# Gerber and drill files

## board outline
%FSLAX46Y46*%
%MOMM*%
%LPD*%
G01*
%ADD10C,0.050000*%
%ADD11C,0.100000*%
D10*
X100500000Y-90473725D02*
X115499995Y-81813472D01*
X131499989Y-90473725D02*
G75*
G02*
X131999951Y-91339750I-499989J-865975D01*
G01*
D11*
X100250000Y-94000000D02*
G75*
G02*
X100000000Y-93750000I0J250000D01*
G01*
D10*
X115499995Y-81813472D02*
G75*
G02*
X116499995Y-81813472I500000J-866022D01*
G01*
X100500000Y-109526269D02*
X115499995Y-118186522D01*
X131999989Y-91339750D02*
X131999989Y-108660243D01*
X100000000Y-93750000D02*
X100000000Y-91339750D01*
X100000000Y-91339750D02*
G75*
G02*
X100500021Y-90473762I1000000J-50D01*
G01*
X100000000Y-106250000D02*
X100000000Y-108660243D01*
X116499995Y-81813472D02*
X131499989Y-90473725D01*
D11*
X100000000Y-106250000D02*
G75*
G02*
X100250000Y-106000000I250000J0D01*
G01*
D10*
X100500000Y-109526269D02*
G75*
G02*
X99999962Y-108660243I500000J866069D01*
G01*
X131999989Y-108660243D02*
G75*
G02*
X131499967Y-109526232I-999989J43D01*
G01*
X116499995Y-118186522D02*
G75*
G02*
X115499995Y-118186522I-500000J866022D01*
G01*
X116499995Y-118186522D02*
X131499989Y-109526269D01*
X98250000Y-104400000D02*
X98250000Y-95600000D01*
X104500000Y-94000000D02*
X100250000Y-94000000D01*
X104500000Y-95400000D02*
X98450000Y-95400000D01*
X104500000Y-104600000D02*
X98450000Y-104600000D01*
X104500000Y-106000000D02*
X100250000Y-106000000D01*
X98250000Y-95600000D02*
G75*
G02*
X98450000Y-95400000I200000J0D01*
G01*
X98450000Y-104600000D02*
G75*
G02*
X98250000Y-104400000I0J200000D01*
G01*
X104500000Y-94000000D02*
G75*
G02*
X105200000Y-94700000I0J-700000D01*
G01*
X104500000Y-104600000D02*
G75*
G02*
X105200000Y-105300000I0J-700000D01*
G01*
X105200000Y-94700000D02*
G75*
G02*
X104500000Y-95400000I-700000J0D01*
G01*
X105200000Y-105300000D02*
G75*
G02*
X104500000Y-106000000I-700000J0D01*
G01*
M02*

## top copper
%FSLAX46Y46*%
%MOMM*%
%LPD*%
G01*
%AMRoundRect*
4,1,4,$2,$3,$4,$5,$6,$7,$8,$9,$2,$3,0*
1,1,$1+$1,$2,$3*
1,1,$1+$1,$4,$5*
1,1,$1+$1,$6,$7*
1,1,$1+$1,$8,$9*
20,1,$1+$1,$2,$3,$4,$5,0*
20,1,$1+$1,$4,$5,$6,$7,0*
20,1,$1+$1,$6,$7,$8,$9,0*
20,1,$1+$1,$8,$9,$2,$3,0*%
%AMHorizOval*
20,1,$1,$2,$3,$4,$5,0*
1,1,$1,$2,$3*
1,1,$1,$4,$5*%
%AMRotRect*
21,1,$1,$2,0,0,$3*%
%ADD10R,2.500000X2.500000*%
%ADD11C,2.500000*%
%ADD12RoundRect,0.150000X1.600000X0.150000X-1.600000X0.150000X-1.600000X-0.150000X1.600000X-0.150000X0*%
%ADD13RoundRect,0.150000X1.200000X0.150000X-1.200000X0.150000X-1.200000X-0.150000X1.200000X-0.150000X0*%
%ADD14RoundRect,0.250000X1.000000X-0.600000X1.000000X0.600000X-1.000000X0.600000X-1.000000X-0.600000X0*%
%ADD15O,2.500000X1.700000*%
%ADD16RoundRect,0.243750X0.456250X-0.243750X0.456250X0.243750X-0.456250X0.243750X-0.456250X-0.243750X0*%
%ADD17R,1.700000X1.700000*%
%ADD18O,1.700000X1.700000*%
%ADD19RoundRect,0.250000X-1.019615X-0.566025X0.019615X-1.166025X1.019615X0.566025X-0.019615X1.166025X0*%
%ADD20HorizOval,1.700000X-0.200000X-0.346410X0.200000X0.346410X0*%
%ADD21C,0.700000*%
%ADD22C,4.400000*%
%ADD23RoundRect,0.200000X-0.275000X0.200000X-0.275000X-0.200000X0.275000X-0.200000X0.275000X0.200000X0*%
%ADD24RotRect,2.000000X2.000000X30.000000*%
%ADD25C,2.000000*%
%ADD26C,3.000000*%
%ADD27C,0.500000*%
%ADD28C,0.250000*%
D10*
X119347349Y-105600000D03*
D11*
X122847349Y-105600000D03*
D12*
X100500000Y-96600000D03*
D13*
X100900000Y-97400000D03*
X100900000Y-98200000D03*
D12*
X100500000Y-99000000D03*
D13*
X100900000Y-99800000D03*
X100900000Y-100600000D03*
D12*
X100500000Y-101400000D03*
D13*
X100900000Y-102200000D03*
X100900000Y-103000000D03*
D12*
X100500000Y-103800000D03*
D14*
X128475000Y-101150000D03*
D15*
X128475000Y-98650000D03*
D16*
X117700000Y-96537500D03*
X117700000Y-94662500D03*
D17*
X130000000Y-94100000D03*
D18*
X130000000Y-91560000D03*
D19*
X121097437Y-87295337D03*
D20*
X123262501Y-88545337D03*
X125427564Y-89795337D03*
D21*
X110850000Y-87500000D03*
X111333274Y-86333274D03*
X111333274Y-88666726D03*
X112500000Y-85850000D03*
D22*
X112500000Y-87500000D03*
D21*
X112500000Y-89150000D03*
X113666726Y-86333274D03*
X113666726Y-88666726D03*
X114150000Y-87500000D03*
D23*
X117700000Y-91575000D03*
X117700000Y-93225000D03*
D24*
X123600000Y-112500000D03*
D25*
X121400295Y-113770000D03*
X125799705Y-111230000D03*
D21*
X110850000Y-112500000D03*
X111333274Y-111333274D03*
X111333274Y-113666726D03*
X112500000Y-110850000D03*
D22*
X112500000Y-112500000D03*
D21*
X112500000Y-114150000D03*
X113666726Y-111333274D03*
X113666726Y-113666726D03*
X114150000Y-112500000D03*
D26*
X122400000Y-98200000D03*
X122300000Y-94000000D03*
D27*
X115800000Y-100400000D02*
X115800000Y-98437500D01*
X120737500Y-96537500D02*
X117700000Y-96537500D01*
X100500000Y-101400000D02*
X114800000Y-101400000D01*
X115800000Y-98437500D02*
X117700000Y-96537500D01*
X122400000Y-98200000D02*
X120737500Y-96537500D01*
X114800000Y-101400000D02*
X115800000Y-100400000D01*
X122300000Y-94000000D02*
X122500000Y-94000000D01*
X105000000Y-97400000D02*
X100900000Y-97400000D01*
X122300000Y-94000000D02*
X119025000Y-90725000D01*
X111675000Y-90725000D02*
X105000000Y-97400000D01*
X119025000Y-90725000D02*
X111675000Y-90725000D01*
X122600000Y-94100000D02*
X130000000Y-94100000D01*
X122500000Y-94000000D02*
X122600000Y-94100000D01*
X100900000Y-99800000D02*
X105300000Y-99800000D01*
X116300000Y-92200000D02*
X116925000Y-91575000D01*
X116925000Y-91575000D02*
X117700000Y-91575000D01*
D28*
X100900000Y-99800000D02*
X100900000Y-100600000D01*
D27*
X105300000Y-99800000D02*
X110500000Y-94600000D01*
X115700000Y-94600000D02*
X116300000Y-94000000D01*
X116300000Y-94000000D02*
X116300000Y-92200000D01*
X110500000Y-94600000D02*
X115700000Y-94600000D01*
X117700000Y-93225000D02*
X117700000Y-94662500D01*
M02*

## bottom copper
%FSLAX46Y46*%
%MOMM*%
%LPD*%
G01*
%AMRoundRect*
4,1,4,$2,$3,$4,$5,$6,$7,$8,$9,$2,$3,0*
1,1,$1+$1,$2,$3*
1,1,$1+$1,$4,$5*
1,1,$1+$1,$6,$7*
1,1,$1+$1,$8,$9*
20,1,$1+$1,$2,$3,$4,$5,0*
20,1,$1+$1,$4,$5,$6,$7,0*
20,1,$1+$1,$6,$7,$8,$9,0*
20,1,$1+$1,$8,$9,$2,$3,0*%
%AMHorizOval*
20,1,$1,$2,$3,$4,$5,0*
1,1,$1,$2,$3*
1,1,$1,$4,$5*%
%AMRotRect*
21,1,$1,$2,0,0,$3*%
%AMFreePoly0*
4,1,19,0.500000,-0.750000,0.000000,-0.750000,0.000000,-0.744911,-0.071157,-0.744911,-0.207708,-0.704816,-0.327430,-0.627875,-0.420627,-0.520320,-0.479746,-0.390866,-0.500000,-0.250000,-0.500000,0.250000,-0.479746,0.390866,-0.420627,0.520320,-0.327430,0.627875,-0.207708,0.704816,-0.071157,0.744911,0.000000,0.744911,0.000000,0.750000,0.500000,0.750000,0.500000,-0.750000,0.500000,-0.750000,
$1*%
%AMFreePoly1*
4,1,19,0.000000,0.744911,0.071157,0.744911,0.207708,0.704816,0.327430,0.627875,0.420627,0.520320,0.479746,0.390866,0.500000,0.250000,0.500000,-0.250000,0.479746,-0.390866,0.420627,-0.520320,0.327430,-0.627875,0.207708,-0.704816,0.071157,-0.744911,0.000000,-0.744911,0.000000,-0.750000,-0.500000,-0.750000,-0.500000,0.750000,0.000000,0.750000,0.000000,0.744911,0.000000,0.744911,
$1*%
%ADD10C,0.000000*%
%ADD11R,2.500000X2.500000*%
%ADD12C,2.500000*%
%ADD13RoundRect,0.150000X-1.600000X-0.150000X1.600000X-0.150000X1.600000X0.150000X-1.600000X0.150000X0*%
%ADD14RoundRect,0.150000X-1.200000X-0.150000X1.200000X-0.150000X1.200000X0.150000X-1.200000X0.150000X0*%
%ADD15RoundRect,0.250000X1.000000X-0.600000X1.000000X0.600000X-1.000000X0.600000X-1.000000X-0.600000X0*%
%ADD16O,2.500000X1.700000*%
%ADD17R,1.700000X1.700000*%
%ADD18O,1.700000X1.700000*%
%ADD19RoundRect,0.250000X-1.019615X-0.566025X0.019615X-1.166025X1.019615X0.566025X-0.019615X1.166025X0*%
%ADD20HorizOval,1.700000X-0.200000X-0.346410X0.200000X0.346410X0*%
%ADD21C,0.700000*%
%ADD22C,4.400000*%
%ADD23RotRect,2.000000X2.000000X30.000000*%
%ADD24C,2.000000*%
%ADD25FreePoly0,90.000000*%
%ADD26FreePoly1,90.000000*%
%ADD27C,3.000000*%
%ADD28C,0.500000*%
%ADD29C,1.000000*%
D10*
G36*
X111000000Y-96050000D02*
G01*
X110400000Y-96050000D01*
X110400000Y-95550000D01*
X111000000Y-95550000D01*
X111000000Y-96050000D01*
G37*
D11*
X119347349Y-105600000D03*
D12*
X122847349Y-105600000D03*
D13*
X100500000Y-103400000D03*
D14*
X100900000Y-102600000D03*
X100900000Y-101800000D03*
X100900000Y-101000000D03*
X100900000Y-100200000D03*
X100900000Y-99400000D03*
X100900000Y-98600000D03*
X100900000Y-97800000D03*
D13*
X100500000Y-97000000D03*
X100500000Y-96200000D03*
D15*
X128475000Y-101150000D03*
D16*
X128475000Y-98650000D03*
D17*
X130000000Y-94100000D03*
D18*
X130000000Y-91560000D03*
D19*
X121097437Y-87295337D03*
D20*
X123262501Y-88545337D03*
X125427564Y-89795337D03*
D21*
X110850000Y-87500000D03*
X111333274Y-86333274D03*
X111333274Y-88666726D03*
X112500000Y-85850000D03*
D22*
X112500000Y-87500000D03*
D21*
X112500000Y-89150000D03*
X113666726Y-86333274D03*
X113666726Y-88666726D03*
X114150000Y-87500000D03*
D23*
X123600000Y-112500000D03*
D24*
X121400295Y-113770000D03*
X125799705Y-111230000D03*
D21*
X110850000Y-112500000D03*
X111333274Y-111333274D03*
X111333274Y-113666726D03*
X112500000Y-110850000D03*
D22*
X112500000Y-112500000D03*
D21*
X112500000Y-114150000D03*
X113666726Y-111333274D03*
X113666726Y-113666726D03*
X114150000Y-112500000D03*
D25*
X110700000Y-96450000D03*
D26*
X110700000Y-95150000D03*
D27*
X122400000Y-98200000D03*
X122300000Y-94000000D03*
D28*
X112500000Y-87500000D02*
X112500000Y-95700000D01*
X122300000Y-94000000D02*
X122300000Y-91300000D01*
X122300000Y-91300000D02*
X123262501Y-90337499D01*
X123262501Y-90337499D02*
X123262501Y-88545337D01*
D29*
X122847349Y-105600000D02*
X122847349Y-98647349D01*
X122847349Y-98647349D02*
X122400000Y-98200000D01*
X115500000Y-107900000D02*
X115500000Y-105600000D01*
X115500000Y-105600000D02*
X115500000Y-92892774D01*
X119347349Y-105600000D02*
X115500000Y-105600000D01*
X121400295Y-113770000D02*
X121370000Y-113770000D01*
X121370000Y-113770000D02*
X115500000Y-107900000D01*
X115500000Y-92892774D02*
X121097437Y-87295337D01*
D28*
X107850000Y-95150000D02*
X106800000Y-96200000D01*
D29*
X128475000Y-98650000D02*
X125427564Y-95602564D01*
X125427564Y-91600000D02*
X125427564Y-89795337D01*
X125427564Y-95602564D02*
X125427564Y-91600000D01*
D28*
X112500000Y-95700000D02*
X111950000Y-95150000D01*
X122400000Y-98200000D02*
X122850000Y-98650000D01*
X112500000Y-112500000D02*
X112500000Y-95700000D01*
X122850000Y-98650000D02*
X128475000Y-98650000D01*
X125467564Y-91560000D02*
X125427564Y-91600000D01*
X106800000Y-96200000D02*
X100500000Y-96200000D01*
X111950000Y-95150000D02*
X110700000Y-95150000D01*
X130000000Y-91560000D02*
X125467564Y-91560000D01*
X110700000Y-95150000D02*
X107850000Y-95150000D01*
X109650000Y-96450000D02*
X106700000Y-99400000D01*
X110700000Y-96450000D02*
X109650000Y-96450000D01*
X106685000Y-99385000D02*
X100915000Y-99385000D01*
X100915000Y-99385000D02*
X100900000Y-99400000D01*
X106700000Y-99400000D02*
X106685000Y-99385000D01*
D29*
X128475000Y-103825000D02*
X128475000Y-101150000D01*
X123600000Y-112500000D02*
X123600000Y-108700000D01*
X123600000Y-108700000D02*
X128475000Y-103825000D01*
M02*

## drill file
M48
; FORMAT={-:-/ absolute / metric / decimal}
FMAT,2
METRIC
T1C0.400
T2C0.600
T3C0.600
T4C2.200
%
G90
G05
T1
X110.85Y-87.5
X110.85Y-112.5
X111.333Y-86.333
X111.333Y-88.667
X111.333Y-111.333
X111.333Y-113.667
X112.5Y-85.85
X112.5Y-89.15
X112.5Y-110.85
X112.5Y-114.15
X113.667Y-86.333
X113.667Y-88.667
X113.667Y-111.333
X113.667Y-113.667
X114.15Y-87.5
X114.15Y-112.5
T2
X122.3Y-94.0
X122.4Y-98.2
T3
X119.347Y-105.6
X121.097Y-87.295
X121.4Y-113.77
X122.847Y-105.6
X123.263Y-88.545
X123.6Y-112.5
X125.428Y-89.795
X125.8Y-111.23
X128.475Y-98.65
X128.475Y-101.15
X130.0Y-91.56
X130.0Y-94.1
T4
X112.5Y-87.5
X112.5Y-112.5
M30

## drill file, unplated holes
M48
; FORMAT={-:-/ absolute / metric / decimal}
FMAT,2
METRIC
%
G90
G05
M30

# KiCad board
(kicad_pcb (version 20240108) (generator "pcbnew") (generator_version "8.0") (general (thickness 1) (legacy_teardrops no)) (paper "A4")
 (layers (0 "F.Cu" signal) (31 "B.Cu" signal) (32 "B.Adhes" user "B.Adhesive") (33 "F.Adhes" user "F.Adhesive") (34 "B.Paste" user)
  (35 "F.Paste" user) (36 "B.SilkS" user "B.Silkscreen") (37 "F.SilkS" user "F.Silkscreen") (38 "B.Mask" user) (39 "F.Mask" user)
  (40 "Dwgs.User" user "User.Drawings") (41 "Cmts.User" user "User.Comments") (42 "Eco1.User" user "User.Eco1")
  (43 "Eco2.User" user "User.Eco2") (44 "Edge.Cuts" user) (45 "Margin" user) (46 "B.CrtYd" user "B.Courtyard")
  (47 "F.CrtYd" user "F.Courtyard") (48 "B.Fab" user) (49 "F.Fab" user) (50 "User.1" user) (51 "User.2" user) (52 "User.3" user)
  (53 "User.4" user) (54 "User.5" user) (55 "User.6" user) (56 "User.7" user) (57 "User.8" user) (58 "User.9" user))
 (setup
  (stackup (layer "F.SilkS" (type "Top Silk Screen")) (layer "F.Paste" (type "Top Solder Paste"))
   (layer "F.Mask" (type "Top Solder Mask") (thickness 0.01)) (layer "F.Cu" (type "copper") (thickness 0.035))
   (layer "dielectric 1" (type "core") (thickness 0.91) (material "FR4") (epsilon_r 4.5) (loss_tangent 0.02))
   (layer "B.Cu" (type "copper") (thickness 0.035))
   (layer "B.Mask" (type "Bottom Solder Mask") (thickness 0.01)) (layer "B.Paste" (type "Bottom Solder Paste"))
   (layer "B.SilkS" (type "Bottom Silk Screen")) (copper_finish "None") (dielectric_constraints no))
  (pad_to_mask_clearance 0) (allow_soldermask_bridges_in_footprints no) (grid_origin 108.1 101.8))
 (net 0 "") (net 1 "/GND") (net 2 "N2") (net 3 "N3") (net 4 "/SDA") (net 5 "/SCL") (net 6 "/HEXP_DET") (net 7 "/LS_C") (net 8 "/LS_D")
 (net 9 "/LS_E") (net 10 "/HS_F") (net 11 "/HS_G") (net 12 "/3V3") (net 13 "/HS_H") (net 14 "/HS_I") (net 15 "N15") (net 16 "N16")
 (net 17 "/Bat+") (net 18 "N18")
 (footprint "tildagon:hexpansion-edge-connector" (layer "F.Cu") (at 98.25 100)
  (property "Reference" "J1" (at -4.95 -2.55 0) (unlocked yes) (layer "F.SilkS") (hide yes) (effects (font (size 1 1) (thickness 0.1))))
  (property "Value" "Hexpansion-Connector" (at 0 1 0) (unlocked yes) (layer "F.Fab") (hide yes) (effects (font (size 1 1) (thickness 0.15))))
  (fp_line (start 0 4.4) (end 0 -4.4) (stroke (width 0.05) (type solid)) (layer "Edge.Cuts"))
  (fp_line (start 6.25 -6) (end 2 -6) (stroke (width 0.05) (type solid)) (layer "Edge.Cuts"))
  (fp_line (start 6.25 -4.6) (end 0.2 -4.6) (stroke (width 0.05) (type solid)) (layer "Edge.Cuts"))
  (fp_line (start 6.25 4.6) (end 0.2 4.6) (stroke (width 0.05) (type solid)) (layer "Edge.Cuts"))
  (fp_line (start 6.25 6) (end 2 6) (stroke (width 0.05) (type solid)) (layer "Edge.Cuts"))
  (fp_arc (start 0 -4.4) (mid 0.058579 -4.541421) (end 0.2 -4.6) (stroke (width 0.05) (type default)) (layer "Edge.Cuts"))
  (fp_arc (start 0.2 4.6) (mid 0.058579 4.541421) (end 0 4.4) (stroke (width 0.05) (type default)) (layer "Edge.Cuts"))
  (fp_arc (start 6.25 -6) (mid 6.744975 -5.794975) (end 6.95 -5.3) (stroke (width 0.05) (type default)) (layer "Edge.Cuts"))
  (fp_arc (start 6.25 4.6) (mid 6.744975 4.805025) (end 6.95 5.3) (stroke (width 0.05) (type default)) (layer "Edge.Cuts"))
  (fp_arc (start 6.95 -5.3) (mid 6.744975 -4.805025) (end 6.25 -4.6) (stroke (width 0.05) (type default)) (layer "Edge.Cuts"))
  (fp_arc (start 6.95 5.3) (mid 6.744975 5.794975) (end 6.25 6) (stroke (width 0.05) (type default)) (layer "Edge.Cuts"))
  (pad "1" smd roundrect (at 2.25 3.4) (size 3.5 0.6) (layers "B.Cu" "B.Mask") (roundrect_rratio 0.25) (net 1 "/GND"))
  (pad "2" smd roundrect (at 2.65 2.6) (size 2.7 0.6) (layers "B.Cu" "B.Mask") (roundrect_rratio 0.25) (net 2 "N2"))
  (pad "3" smd roundrect (at 2.65 1.8) (size 2.7 0.6) (layers "B.Cu" "B.Mask") (roundrect_rratio 0.25) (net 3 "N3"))
  (pad "4" smd roundrect (at 2.65 1) (size 2.7 0.6) (layers "B.Cu" "B.Mask") (roundrect_rratio 0.25) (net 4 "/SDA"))
  (pad "5" smd roundrect (at 2.65 0.2) (size 2.7 0.6) (layers "B.Cu" "B.Mask") (roundrect_rratio 0.25) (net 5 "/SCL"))
  (pad "6" smd roundrect (at 2.65 -0.6) (size 2.7 0.6) (layers "B.Cu" "B.Mask") (roundrect_rratio 0.25) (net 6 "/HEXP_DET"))
  (pad "7" smd roundrect (at 2.65 -1.4) (size 2.7 0.6) (layers "B.Cu" "B.Mask") (roundrect_rratio 0.25) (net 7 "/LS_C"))
  (pad "8" smd roundrect (at 2.65 -2.2) (size 2.7 0.6) (layers "B.Cu" "B.Mask") (roundrect_rratio 0.25) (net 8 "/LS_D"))
  (pad "9" smd roundrect (at 2.25 -3) (size 3.5 0.6) (layers "B.Cu" "B.Mask") (roundrect_rratio 0.25) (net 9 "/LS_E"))
  (pad "10" smd roundrect (at 2.25 -3.8) (size 3.5 0.6) (layers "B.Cu" "B.Mask") (roundrect_rratio 0.25) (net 1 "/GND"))
  (pad "11" smd roundrect (at 2.25 -3.4 180) (size 3.5 0.6) (layers "F.Cu" "F.Mask") (roundrect_rratio 0.25) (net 1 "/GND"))
  (pad "12" smd roundrect (at 2.65 -2.6 180) (size 2.7 0.6) (layers "F.Cu" "F.Mask") (roundrect_rratio 0.25) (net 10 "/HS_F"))
  (pad "13" smd roundrect (at 2.65 -1.8 180) (size 2.7 0.6) (layers "F.Cu" "F.Mask") (roundrect_rratio 0.25) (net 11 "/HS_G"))
  (pad "14" smd roundrect (at 2.25 -1 180) (size 3.5 0.6) (layers "F.Cu" "F.Mask") (roundrect_rratio 0.25) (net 1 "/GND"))
  (pad "15" smd roundrect (at 2.65 -0.2 180) (size 2.7 0.6) (layers "F.Cu" "F.Mask") (roundrect_rratio 0.25) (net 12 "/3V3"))
  (pad "16" smd roundrect (at 2.65 0.6 180) (size 2.7 0.6) (layers "F.Cu" "F.Mask") (roundrect_rratio 0.25) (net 12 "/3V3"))
  (pad "17" smd roundrect (at 2.25 1.4 180) (size 3.5 0.6) (layers "F.Cu" "F.Mask") (roundrect_rratio 0.25) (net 1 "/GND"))
  (pad "18" smd roundrect (at 2.65 2.2 180) (size 2.7 0.6) (layers "F.Cu" "F.Mask") (roundrect_rratio 0.25) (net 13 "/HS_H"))
  (pad "19" smd roundrect (at 2.65 3 180) (size 2.7 0.6) (layers "F.Cu" "F.Mask") (roundrect_rratio 0.25) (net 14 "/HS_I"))
  (pad "20" smd roundrect (at 2.25 3.8 180) (size 3.5 0.6) (layers "F.Cu" "F.Mask") (roundrect_rratio 0.25) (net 1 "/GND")))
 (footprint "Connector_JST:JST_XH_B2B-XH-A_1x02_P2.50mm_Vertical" (layer "F.Cu") (at 128.475 101.15 90)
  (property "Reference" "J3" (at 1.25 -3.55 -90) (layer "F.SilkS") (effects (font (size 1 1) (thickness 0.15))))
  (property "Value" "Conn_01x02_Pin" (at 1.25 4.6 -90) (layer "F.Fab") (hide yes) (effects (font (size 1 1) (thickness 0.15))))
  (pad "1" thru_hole roundrect (at 0 0 90) (size 1.7 2.5) (drill 0.6) (layers "*.Cu" "*.Mask") (remove_unused_layers no)
   (roundrect_rratio 0.147059) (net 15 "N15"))
  (pad "2" thru_hole oval (at 2.5 0 90) (size 1.7 2.5) (drill 0.6) (layers "*.Cu" "*.Mask") (remove_unused_layers no) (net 1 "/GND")))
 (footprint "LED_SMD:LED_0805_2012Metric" (layer "F.Cu") (at 117.7 95.6 90)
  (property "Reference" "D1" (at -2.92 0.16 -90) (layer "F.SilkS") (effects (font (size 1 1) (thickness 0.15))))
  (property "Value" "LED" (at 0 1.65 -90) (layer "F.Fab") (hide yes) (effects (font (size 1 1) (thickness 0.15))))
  (pad "1" smd roundrect (at -0.9375 0 90) (size 0.975 1.4) (layers "F.Cu" "F.Paste" "F.Mask") (roundrect_rratio 0.25) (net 1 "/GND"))
  (pad "2" smd roundrect (at 0.9375 0 90) (size 0.975 1.4) (layers "F.Cu" "F.Paste" "F.Mask") (roundrect_rratio 0.25) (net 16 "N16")))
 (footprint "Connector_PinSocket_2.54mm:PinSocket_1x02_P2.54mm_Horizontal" (layer "F.Cu") (at 130 94.1 180)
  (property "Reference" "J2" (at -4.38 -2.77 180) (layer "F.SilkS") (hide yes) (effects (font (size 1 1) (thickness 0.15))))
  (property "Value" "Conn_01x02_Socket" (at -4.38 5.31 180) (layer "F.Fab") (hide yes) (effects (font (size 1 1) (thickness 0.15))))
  (pad "1" thru_hole rect (at 0 0 180) (size 1.7 1.7) (drill 0.6) (layers "*.Cu" "*.Mask") (remove_unused_layers no) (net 10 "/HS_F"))
  (pad "2" thru_hole oval (at 0 2.54 180) (size 1.7 1.7) (drill 0.6) (layers "*.Cu" "*.Mask") (remove_unused_layers no) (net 1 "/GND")))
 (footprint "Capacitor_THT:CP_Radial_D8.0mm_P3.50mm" (layer "F.Cu") (at 119.347349 105.6)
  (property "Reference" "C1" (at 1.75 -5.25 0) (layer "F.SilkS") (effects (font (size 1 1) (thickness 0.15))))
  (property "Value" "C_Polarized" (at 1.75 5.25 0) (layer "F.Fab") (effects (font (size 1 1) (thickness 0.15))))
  (pad "1" thru_hole rect (at 0 0) (size 2.5 2.5) (drill 0.6) (layers "*.Cu" "*.Mask") (remove_unused_layers no) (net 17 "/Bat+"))
  (pad "2" thru_hole circle (at 3.5 0) (size 2.5 2.5) (drill 0.6) (layers "*.Cu" "*.Mask") (remove_unused_layers no) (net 1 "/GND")))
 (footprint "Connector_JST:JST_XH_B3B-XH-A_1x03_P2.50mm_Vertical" (layer "F.Cu") (at 121.097437 87.295337 -30)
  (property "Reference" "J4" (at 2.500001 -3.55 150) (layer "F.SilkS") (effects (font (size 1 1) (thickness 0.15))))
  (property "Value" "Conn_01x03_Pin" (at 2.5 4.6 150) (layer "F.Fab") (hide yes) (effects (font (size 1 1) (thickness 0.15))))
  (pad "1" thru_hole roundrect (at 0 0 330) (size 1.7 2.5) (drill 0.6) (layers "*.Cu" "*.Mask") (remove_unused_layers no)
   (roundrect_rratio 0.147059) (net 17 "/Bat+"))
  (pad "2" thru_hole oval (at 2.5 0 330) (size 1.7 2.5) (drill 0.6) (layers "*.Cu" "*.Mask") (remove_unused_layers no) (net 10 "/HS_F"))
  (pad "3" thru_hole oval (at 5 0 330) (size 1.7 2.5) (drill 0.6) (layers "*.Cu" "*.Mask") (remove_unused_layers no) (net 1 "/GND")))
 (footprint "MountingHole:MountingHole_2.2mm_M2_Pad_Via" (layer "F.Cu") (at 112.5 87.5)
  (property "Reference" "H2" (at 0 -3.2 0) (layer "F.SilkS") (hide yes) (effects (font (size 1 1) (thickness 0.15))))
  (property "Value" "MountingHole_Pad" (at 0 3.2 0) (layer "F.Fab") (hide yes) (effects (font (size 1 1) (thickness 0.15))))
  (pad "1" thru_hole circle (at -1.65 0) (size 0.7 0.7) (drill 0.4) (layers "*.Cu" "*.Mask") (remove_unused_layers no) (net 1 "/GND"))
  (pad "1" thru_hole circle (at -1.166726 -1.166726) (size 0.7 0.7) (drill 0.4) (layers "*.Cu" "*.Mask") (remove_unused_layers no)
   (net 1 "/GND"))
  (pad "1" thru_hole circle (at -1.166726 1.166726) (size 0.7 0.7) (drill 0.4) (layers "*.Cu" "*.Mask") (remove_unused_layers no)
   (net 1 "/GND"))
  (pad "1" thru_hole circle (at 0 -1.65) (size 0.7 0.7) (drill 0.4) (layers "*.Cu" "*.Mask") (remove_unused_layers no) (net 1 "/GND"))
  (pad "1" thru_hole circle (at 0 0) (size 4.4 4.4) (drill 2.2) (layers "*.Cu" "*.Mask") (remove_unused_layers no) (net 1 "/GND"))
  (pad "1" thru_hole circle (at 0 1.65) (size 0.7 0.7) (drill 0.4) (layers "*.Cu" "*.Mask") (remove_unused_layers no) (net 1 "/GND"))
  (pad "1" thru_hole circle (at 1.166726 -1.166726) (size 0.7 0.7) (drill 0.4) (layers "*.Cu" "*.Mask") (remove_unused_layers no)
   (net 1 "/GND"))
  (pad "1" thru_hole circle (at 1.166726 1.166726) (size 0.7 0.7) (drill 0.4) (layers "*.Cu" "*.Mask") (remove_unused_layers no)
   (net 1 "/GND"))
  (pad "1" thru_hole circle (at 1.65 0) (size 0.7 0.7) (drill 0.4) (layers "*.Cu" "*.Mask") (remove_unused_layers no) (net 1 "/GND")))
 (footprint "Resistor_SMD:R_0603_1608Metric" (layer "F.Cu") (at 117.7 92.4 -90)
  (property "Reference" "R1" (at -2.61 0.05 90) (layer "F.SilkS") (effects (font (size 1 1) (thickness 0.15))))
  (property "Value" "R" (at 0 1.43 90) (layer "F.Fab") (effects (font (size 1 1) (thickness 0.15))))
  (pad "1" smd roundrect (at -0.825 0 270) (size 0.8 0.95) (layers "F.Cu" "F.Paste" "F.Mask") (roundrect_rratio 0.25) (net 12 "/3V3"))
  (pad "2" smd roundrect (at 0.825 0 270) (size 0.8 0.95) (layers "F.Cu" "F.Paste" "F.Mask") (roundrect_rratio 0.25) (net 16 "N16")))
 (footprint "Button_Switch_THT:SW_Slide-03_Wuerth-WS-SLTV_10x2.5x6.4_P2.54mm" (layer "F.Cu") (at 123.6 112.5 30)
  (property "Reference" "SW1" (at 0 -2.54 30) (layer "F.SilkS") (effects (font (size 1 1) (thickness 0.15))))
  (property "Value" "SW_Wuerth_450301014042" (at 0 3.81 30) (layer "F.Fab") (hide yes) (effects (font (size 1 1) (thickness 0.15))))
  (pad "1" thru_hole rect (at 0 0 30) (size 2 2) (drill 0.6) (layers "*.Cu" "*.Mask") (remove_unused_layers no) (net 15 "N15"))
  (pad "2" thru_hole circle (at -2.54 0 30) (size 2 2) (drill 0.6) (layers "*.Cu" "*.Mask") (remove_unused_layers no) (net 17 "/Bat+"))
  (pad "3" thru_hole circle (at 2.54 0 30) (size 2 2) (drill 0.6) (layers "*.Cu" "*.Mask") (remove_unused_layers no) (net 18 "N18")))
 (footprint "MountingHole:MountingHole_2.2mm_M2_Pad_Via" (layer "F.Cu") (at 112.5 112.5)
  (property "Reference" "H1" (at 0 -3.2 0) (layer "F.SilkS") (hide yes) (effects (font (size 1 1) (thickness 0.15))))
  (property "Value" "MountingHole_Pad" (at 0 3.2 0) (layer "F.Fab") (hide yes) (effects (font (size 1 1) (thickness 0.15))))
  (pad "1" thru_hole circle (at -1.65 0) (size 0.7 0.7) (drill 0.4) (layers "*.Cu" "*.Mask") (remove_unused_layers no) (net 1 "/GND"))
  (pad "1" thru_hole circle (at -1.166726 -1.166726) (size 0.7 0.7) (drill 0.4) (layers "*.Cu" "*.Mask") (remove_unused_layers no)
   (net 1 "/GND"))
  (pad "1" thru_hole circle (at -1.166726 1.166726) (size 0.7 0.7) (drill 0.4) (layers "*.Cu" "*.Mask") (remove_unused_layers no)
   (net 1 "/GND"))
  (pad "1" thru_hole circle (at 0 -1.65) (size 0.7 0.7) (drill 0.4) (layers "*.Cu" "*.Mask") (remove_unused_layers no) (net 1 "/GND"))
  (pad "1" thru_hole circle (at 0 0) (size 4.4 4.4) (drill 2.2) (layers "*.Cu" "*.Mask") (remove_unused_layers no) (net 1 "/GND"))
  (pad "1" thru_hole circle (at 0 1.65) (size 0.7 0.7) (drill 0.4) (layers "*.Cu" "*.Mask") (remove_unused_layers no) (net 1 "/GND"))
  (pad "1" thru_hole circle (at 1.166726 -1.166726) (size 0.7 0.7) (drill 0.4) (layers "*.Cu" "*.Mask") (remove_unused_layers no)
   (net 1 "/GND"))
  (pad "1" thru_hole circle (at 1.166726 1.166726) (size 0.7 0.7) (drill 0.4) (layers "*.Cu" "*.Mask") (remove_unused_layers no)
   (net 1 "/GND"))
  (pad "1" thru_hole circle (at 1.65 0) (size 0.7 0.7) (drill 0.4) (layers "*.Cu" "*.Mask") (remove_unused_layers no) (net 1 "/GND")))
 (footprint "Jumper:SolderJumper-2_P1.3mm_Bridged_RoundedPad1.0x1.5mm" (layer "B.Cu") (at 110.7 95.8 90)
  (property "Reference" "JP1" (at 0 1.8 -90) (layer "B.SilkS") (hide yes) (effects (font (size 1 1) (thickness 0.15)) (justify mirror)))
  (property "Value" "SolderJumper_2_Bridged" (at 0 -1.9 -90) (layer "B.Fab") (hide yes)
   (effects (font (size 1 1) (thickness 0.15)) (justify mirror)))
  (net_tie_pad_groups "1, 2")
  (fp_poly (pts (xy 0.25 0.3) (xy -0.25 0.3) (xy -0.25 -0.3) (xy 0.25 -0.3)) (stroke (width 0) (type solid)) (fill solid) (layer "B.Cu"))
  (pad "1" smd custom (at -0.65 0 90) (size 1 0.5) (layers "B.Cu" "B.Mask") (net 6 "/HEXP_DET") (zone_connect 2)
   (options (clearance outline) (anchor rect)) (primitives))
  (pad "2" smd custom (at 0.65 0 90) (size 1 0.5) (layers "B.Cu" "B.Mask") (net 1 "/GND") (zone_connect 2)
   (options (clearance outline) (anchor rect)) (primitives)))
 (gr_line (start 100.5 90.473725) (end 115.499995 81.813472) (stroke (width 0.05) (type solid)) (layer "Edge.Cuts"))
 (gr_arc (start 131.499989 90.473725) (mid 131.866015 90.83975) (end 131.999989 91.33975) (stroke (width 0.05) (type solid))
  (layer "Edge.Cuts"))
 (gr_arc (start 100.25 94) (mid 100.073223 93.926777) (end 100 93.75) (stroke (width 0.1) (type default)) (layer "Edge.Cuts"))
 (gr_arc (start 115.499995 81.813472) (mid 115.999995 81.679497) (end 116.499995 81.813472) (stroke (width 0.05) (type solid))
  (layer "Edge.Cuts"))
 (gr_line (start 100.5 109.526269) (end 115.499995 118.186522) (stroke (width 0.05) (type solid)) (layer "Edge.Cuts"))
 (gr_line (start 131.999989 91.33975) (end 131.999989 108.660243) (stroke (width 0.05) (type solid)) (layer "Edge.Cuts"))
 (gr_line (start 100 93.75) (end 100 91.33975) (stroke (width 0.05) (type solid)) (layer "Edge.Cuts"))
 (gr_arc (start 100 91.33975) (mid 100.133975 90.83975) (end 100.5 90.473725) (stroke (width 0.05) (type solid)) (layer "Edge.Cuts"))
 (gr_line (start 100 106.25) (end 100 108.660243) (stroke (width 0.05) (type solid)) (layer "Edge.Cuts"))
 (gr_line (start 116.499995 81.813472) (end 131.499989 90.473725) (stroke (width 0.05) (type solid)) (layer "Edge.Cuts"))
 (gr_arc (start 100 106.25) (mid 100.073223 106.073223) (end 100.25 106) (stroke (width 0.1) (type default)) (layer "Edge.Cuts"))
 (gr_arc (start 100.5 109.526269) (mid 100.133975 109.160243) (end 100 108.660243) (stroke (width 0.05) (type solid)) (layer "Edge.Cuts"))
 (gr_arc (start 131.999989 108.660243) (mid 131.866015 109.160243) (end 131.499989 109.526269) (stroke (width 0.05) (type solid))
  (layer "Edge.Cuts"))
 (gr_arc (start 116.499995 118.186522) (mid 115.999995 118.320497) (end 115.499995 118.186522) (stroke (width 0.05) (type solid))
  (layer "Edge.Cuts"))
 (gr_line (start 116.499995 118.186522) (end 131.499989 109.526269) (stroke (width 0.05) (type solid)) (layer "Edge.Cuts"))
 (segment (start 115.8 100.4) (end 115.8 98.4375) (width 0.5) (layer "F.Cu") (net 1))
 (segment (start 120.7375 96.5375) (end 117.7 96.5375) (width 0.5) (layer "F.Cu") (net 1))
 (segment (start 100.5 101.4) (end 114.8 101.4) (width 0.5) (layer "F.Cu") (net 1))
 (segment (start 115.8 98.4375) (end 117.7 96.5375) (width 0.5) (layer "F.Cu") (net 1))
 (segment (start 122.4 98.2) (end 120.7375 96.5375) (width 0.5) (layer "F.Cu") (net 1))
 (segment (start 114.8 101.4) (end 115.8 100.4) (width 0.5) (layer "F.Cu") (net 1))
 (via (at 122.4 98.2) (size 3) (drill 0.6) (layers "F.Cu" "B.Cu") (free yes) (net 1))
 (segment (start 107.85 95.15) (end 106.8 96.2) (width 0.5) (layer "B.Cu") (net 1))
 (segment (start 128.475 98.65) (end 125.427564 95.602564) (width 1) (layer "B.Cu") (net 1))
 (segment (start 125.427564 91.6) (end 125.427564 89.795337) (width 1) (layer "B.Cu") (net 1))
 (segment (start 125.427564 95.602564) (end 125.427564 91.6) (width 1) (layer "B.Cu") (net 1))
 (segment (start 122.847349 98.647349) (end 122.4 98.2) (width 1) (layer "B.Cu") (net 1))
 (segment (start 112.5 95.7) (end 111.95 95.15) (width 0.5) (layer "B.Cu") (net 1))
 (segment (start 122.4 98.2) (end 122.85 98.65) (width 0.5) (layer "B.Cu") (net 1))
 (segment (start 112.5 112.5) (end 112.5 95.7) (width 0.5) (layer "B.Cu") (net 1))
 (segment (start 112.5 87.5) (end 112.5 95.7) (width 0.5) (layer "B.Cu") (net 1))
 (segment (start 122.847349 105.6) (end 122.847349 98.647349) (width 1) (layer "B.Cu") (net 1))
 (segment (start 122.85 98.65) (end 128.475 98.65) (width 0.5) (layer "B.Cu") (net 1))
 (segment (start 125.467564 91.56) (end 125.427564 91.6) (width 0.5) (layer "B.Cu") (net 1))
 (segment (start 106.8 96.2) (end 100.5 96.2) (width 0.5) (layer "B.Cu") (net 1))
 (segment (start 111.95 95.15) (end 110.7 95.15) (width 0.5) (layer "B.Cu") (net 1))
 (segment (start 130 91.56) (end 125.467564 91.56) (width 0.5) (layer "B.Cu") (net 1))
 (segment (start 110.7 95.15) (end 107.85 95.15) (width 0.5) (layer "B.Cu") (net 1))
 (segment (start 122.3 94) (end 122.5 94) (width 0.5) (layer "F.Cu") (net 10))
 (segment (start 105 97.4) (end 100.9 97.4) (width 0.5) (layer "F.Cu") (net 10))
 (segment (start 122.3 94) (end 119.025 90.725) (width 0.5) (layer "F.Cu") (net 10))
 (segment (start 111.675 90.725) (end 105 97.4) (width 0.5) (layer "F.Cu") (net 10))
 (segment (start 119.025 90.725) (end 111.675 90.725) (width 0.5) (layer "F.Cu") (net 10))
 (segment (start 122.6 94.1) (end 130 94.1) (width 0.5) (layer "F.Cu") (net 10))
 (segment (start 122.5 94) (end 122.6 94.1) (width 0.5) (layer "F.Cu") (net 10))
 (via (at 122.3 94) (size 3) (drill 0.6) (layers "F.Cu" "B.Cu") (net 10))
 (segment (start 122.3 91.3) (end 123.262501 90.337499) (width 0.5) (layer "B.Cu") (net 10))
 (segment (start 122.3 94) (end 122.3 91.3) (width 0.5) (layer "B.Cu") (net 10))
 (segment (start 123.262501 90.337499) (end 123.262501 88.545337) (width 0.5) (layer "B.Cu") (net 10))
 (segment (start 100.9 99.8) (end 105.3 99.8) (width 0.5) (layer "F.Cu") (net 12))
 (segment (start 116.3 92.2) (end 116.925 91.575) (width 0.5) (layer "F.Cu") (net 12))
 (segment (start 116.925 91.575) (end 117.7 91.575) (width 0.5) (layer "F.Cu") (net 12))
 (segment (start 100.9 99.8) (end 100.9 100.6) (width 0.25) (layer "F.Cu") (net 12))
 (segment (start 105.3 99.8) (end 110.5 94.6) (width 0.5) (layer "F.Cu") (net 12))
 (segment (start 115.7 94.6) (end 116.3 94) (width 0.5) (layer "F.Cu") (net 12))
 (segment (start 116.3 94) (end 116.3 92.2) (width 0.5) (layer "F.Cu") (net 12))
 (segment (start 110.5 94.6) (end 115.7 94.6) (width 0.5) (layer "F.Cu") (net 12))
 (segment (start 117.7 93.225) (end 117.7 94.6625) (width 0.5) (layer "F.Cu") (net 16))
 (segment (start 109.65 96.45) (end 106.7 99.4) (width 0.5) (layer "B.Cu") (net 6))
 (segment (start 110.7 96.45) (end 109.65 96.45) (width 0.5) (layer "B.Cu") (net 6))
 (segment (start 106.685 99.385) (end 100.915 99.385) (width 0.5) (layer "B.Cu") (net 6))
 (segment (start 100.915 99.385) (end 100.9 99.4) (width 0.5) (layer "B.Cu") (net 6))
 (segment (start 106.7 99.4) (end 106.685 99.385) (width 0.5) (layer "B.Cu") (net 6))
 (segment (start 128.475 103.825) (end 128.475 101.15) (width 1) (layer "B.Cu") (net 15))
 (segment (start 123.6 112.5) (end 123.6 108.7) (width 1) (layer "B.Cu") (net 15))
 (segment (start 123.6 108.7) (end 128.475 103.825) (width 1) (layer "B.Cu") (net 15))
 (segment (start 115.5 105.6) (end 115.5 92.892774) (width 1) (layer "B.Cu") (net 17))
 (segment (start 119.347349 105.6) (end 115.5 105.6) (width 1) (layer "B.Cu") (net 17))
 (segment (start 121.400295 113.77) (end 121.37 113.77) (width 1) (layer "B.Cu") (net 17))
 (segment (start 115.5 107.9) (end 115.5 105.6) (width 1) (layer "B.Cu") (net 17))
 (segment (start 115.5 92.892774) (end 121.097437 87.295337) (width 1) (layer "B.Cu") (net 17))
 (segment (start 121.37 113.77) (end 115.5 107.9) (width 1) (layer "B.Cu") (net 17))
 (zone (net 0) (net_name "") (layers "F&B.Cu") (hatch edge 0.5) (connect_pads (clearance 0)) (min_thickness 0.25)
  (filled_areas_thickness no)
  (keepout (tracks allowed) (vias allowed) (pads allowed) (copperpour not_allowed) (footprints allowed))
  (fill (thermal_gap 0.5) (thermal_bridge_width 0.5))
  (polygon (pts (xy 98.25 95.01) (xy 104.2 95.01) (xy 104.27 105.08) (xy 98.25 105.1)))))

